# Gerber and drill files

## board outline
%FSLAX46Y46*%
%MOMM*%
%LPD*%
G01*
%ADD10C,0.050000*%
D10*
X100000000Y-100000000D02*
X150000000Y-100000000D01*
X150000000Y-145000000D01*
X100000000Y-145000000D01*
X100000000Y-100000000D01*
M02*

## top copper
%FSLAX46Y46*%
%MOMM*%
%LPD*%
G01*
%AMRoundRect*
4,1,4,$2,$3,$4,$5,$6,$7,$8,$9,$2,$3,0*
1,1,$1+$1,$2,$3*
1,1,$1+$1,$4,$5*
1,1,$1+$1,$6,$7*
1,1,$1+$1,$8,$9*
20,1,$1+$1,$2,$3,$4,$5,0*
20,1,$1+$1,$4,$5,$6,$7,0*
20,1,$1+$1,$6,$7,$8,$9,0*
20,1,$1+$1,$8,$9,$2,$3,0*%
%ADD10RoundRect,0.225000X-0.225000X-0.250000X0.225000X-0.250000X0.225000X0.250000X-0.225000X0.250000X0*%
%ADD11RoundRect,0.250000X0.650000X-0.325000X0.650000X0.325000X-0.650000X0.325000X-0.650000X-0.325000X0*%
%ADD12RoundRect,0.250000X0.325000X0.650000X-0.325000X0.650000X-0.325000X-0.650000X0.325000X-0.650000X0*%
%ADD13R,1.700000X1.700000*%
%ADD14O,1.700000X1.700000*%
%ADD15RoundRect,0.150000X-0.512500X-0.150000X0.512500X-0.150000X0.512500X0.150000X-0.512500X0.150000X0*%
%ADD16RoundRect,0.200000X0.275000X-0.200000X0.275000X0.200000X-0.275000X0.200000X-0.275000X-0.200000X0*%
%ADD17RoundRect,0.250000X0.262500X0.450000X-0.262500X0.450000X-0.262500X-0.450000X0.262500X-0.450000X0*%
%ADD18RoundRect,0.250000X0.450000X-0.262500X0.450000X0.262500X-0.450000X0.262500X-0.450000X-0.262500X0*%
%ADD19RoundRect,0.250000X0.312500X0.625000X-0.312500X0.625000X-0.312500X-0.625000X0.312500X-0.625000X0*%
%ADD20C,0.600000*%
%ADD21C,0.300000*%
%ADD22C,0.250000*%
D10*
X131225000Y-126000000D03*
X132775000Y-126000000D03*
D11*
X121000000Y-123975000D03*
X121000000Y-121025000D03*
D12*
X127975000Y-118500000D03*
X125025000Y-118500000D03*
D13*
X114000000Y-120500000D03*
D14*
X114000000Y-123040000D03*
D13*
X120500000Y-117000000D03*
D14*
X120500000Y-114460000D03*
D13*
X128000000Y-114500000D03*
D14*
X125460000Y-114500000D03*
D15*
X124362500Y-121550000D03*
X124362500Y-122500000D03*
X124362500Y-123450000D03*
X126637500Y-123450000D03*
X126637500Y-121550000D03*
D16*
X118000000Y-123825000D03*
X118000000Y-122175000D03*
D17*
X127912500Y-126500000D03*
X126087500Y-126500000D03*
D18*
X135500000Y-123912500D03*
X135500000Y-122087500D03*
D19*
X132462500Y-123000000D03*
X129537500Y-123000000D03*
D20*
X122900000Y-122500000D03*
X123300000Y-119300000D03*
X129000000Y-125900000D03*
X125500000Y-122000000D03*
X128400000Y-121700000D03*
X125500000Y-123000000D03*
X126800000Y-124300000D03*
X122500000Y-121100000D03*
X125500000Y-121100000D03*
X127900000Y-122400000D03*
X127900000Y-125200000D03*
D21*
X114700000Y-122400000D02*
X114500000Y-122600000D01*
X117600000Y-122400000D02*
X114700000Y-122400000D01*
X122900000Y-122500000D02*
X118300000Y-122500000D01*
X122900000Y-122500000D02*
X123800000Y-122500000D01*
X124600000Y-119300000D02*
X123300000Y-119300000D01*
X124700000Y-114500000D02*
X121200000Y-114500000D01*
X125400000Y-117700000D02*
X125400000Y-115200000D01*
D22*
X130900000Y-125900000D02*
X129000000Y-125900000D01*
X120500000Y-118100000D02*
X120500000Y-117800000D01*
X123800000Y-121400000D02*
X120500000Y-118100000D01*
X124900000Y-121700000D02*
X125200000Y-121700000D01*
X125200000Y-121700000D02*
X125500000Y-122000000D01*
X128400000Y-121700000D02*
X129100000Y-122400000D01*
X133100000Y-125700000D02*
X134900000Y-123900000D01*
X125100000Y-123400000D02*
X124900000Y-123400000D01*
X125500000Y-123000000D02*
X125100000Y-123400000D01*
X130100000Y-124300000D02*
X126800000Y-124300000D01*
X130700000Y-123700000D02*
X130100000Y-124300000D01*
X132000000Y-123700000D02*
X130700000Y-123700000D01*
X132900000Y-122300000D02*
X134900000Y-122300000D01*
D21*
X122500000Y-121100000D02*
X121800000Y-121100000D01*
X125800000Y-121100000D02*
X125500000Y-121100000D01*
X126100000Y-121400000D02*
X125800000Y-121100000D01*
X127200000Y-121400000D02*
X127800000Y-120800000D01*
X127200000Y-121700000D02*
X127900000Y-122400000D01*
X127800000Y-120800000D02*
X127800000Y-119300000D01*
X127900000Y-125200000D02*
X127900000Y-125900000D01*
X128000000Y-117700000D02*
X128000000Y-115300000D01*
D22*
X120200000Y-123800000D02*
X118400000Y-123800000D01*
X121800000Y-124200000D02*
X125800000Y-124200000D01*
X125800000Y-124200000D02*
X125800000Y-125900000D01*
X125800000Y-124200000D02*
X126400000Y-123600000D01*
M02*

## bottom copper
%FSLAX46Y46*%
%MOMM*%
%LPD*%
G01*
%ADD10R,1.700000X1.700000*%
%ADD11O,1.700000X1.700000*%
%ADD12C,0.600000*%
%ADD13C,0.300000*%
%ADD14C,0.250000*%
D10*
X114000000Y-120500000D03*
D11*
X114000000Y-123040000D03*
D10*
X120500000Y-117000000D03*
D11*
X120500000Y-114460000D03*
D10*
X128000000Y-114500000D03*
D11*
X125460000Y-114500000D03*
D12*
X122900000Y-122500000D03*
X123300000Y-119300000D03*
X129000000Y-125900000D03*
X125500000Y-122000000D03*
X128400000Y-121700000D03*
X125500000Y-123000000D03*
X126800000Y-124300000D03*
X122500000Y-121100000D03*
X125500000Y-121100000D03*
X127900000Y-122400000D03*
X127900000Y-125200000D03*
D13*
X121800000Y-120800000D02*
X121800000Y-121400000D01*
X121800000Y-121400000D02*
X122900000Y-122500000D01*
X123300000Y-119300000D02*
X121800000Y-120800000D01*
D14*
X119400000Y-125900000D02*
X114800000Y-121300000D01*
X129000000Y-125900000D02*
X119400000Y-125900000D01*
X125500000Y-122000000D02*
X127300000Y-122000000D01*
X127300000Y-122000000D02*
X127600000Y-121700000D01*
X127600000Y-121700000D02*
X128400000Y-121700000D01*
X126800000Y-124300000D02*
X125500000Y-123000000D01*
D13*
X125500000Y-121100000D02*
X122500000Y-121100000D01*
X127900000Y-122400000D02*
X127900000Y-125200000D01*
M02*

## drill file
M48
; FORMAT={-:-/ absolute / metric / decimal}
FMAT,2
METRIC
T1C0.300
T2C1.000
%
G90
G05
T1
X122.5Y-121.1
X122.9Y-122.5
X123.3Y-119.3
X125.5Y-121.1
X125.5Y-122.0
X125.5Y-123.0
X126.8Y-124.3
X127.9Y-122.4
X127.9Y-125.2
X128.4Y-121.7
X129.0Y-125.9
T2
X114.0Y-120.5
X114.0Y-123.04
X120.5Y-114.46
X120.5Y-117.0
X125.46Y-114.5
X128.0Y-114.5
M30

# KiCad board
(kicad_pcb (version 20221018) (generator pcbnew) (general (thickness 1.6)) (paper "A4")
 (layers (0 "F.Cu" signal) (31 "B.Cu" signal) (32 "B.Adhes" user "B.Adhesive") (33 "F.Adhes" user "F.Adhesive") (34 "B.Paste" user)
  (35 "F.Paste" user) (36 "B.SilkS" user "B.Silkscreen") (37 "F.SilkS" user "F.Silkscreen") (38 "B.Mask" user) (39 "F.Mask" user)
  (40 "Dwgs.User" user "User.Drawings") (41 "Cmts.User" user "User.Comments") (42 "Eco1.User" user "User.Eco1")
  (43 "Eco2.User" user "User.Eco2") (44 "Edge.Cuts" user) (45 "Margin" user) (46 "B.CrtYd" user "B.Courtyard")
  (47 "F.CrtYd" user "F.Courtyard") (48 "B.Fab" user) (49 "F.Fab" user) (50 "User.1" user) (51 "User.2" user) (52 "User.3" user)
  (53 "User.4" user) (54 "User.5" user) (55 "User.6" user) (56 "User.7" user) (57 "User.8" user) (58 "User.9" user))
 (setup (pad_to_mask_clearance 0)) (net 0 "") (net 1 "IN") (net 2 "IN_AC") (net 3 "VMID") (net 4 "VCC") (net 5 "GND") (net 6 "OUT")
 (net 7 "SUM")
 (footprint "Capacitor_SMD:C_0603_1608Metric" (layer "F.Cu") (at 132 126)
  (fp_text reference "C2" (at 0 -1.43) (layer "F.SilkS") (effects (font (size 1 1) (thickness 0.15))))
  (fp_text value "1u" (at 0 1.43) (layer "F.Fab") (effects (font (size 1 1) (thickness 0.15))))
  (pad "1" smd roundrect (at -0.775 0) (size 0.9 0.95) (layers "F.Cu" "F.Paste" "F.Mask") (roundrect_rratio 0.25) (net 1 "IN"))
  (pad "2" smd roundrect (at 0.775 0) (size 0.9 0.95) (layers "F.Cu" "F.Paste" "F.Mask") (roundrect_rratio 0.25) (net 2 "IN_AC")))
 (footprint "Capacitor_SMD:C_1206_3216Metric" (layer "F.Cu") (at 121 122.5 90)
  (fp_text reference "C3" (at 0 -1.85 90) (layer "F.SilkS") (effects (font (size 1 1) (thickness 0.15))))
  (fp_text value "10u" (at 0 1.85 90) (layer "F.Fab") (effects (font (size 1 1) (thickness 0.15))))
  (pad "1" smd roundrect (at -1.475 0 90) (size 1.15 1.8) (layers "F.Cu" "F.Paste" "F.Mask") (roundrect_rratio 0.217391) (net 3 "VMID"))
  (pad "2" smd roundrect (at 1.475 0 90) (size 1.15 1.8) (layers "F.Cu" "F.Paste" "F.Mask") (roundrect_rratio 0.217391) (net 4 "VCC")))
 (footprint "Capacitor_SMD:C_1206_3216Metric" (layer "F.Cu") (at 126.5 118.5 180)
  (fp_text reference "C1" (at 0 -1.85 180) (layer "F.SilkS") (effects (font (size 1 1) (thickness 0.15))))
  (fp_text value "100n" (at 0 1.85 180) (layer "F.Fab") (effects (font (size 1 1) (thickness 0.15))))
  (pad "1" smd roundrect (at -1.475 0 180) (size 1.15 1.8) (layers "F.Cu" "F.Paste" "F.Mask") (roundrect_rratio 0.217391) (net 4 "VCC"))
  (pad "2" smd roundrect (at 1.475 0 180) (size 1.15 1.8) (layers "F.Cu" "F.Paste" "F.Mask") (roundrect_rratio 0.217391) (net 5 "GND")))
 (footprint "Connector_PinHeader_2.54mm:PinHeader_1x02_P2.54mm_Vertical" (layer "F.Cu") (at 114 120.5)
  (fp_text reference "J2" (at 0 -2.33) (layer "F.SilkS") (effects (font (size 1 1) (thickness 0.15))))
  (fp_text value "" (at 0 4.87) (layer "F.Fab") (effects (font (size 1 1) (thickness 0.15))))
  (pad "1" thru_hole rect (at 0 0) (size 1.7 1.7) (drill 1) (layers "*.Cu" "*.Mask") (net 1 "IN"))
  (pad "2" thru_hole oval (at 0 2.54) (size 1.7 1.7) (drill 1) (layers "*.Cu" "*.Mask") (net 5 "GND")))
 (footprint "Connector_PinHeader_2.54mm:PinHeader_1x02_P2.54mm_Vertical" (layer "F.Cu") (at 120.5 117 180)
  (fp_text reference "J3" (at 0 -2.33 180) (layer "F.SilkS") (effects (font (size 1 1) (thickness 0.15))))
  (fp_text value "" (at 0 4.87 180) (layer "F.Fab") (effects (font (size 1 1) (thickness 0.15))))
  (pad "1" thru_hole rect (at 0 0 180) (size 1.7 1.7) (drill 1) (layers "*.Cu" "*.Mask") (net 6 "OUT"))
  (pad "2" thru_hole oval (at 0 2.54 180) (size 1.7 1.7) (drill 1) (layers "*.Cu" "*.Mask") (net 5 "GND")))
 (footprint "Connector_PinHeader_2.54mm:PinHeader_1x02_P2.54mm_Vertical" (layer "F.Cu") (at 128 114.5 -90)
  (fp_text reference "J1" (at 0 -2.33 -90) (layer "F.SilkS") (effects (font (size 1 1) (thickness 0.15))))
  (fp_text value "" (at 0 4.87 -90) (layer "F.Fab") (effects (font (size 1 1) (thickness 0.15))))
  (pad "1" thru_hole rect (at 0 0 270) (size 1.7 1.7) (drill 1) (layers "*.Cu" "*.Mask") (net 4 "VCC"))
  (pad "2" thru_hole oval (at 0 2.54 270) (size 1.7 1.7) (drill 1) (layers "*.Cu" "*.Mask") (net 5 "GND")))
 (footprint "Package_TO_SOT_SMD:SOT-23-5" (layer "F.Cu") (at 125.5 122.5)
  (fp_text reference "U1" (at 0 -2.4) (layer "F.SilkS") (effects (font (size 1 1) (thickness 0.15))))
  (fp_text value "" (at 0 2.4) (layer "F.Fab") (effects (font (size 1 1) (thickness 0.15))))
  (pad "1" smd roundrect (at -1.1375 -0.95) (size 1.325 0.6) (layers "F.Cu" "F.Paste" "F.Mask") (roundrect_rratio 0.25) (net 6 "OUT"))
  (pad "2" smd roundrect (at -1.1375 0) (size 1.325 0.6) (layers "F.Cu" "F.Paste" "F.Mask") (roundrect_rratio 0.25) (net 5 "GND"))
  (pad "3" smd roundrect (at -1.1375 0.95) (size 1.325 0.6) (layers "F.Cu" "F.Paste" "F.Mask") (roundrect_rratio 0.25) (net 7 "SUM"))
  (pad "4" smd roundrect (at 1.1375 0.95) (size 1.325 0.6) (layers "F.Cu" "F.Paste" "F.Mask") (roundrect_rratio 0.25) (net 3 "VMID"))
  (pad "5" smd roundrect (at 1.1375 -0.95) (size 1.325 0.6) (layers "F.Cu" "F.Paste" "F.Mask") (roundrect_rratio 0.25) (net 4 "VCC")))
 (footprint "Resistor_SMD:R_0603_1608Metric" (layer "F.Cu") (at 118 123 90)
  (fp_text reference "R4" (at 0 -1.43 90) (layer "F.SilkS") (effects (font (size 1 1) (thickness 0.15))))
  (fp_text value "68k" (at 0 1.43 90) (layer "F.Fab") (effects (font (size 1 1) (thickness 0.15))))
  (pad "1" smd roundrect (at -0.825 0 90) (size 0.8 0.95) (layers "F.Cu" "F.Paste" "F.Mask") (roundrect_rratio 0.25) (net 3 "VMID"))
  (pad "2" smd roundrect (at 0.825 0 90) (size 0.8 0.95) (layers "F.Cu" "F.Paste" "F.Mask") (roundrect_rratio 0.25) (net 5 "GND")))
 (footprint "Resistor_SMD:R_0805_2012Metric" (layer "F.Cu") (at 127 126.5 180)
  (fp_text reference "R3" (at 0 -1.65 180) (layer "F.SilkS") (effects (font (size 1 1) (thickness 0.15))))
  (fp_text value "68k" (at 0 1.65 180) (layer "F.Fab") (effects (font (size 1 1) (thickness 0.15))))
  (pad "1" smd roundrect (at -0.9125 0 180) (size 1.025 1.4) (layers "F.Cu" "F.Paste" "F.Mask") (roundrect_rratio 0.243902) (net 4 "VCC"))
  (pad "2" smd roundrect (at 0.9125 0 180) (size 1.025 1.4) (layers "F.Cu" "F.Paste" "F.Mask") (roundrect_rratio 0.243902) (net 3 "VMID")))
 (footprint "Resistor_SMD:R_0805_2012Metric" (layer "F.Cu") (at 135.5 123 90)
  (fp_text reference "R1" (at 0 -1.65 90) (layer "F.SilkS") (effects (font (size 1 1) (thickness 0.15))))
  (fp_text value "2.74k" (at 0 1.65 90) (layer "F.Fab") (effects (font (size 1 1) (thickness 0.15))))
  (pad "1" smd roundrect (at -0.9125 0 90) (size 1.025 1.4) (layers "F.Cu" "F.Paste" "F.Mask") (roundrect_rratio 0.243902) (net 2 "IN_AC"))
  (pad "2" smd roundrect (at 0.9125 0 90) (size 1.025 1.4) (layers "F.Cu" "F.Paste" "F.Mask") (roundrect_rratio 0.243902) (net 7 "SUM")))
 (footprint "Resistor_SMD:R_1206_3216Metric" (layer "F.Cu") (at 131 123 180)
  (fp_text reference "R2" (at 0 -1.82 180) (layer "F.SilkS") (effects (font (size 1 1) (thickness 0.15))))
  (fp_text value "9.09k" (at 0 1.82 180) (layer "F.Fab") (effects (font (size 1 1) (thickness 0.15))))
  (pad "1" smd roundrect (at -1.4625 0 180) (size 1.125 1.75) (layers "F.Cu" "F.Paste" "F.Mask") (roundrect_rratio 0.222222) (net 7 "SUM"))
  (pad "2" smd roundrect (at 1.4625 0 180) (size 1.125 1.75) (layers "F.Cu" "F.Paste" "F.Mask") (roundrect_rratio 0.222222) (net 6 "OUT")))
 (gr_rect (start 100 100) (end 150 145) (stroke (width 0.05) (type default)) (fill none) (layer "Edge.Cuts"))
 (segment (start 114.7 122.4) (end 114.5 122.6) (width 0.3) (layer "F.Cu") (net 5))
 (segment (start 117.6 122.4) (end 114.7 122.4) (width 0.3) (layer "F.Cu") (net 5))
 (segment (start 122.9 122.5) (end 118.3 122.5) (width 0.3) (layer "F.Cu") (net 5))
 (segment (start 122.9 122.5) (end 123.8 122.5) (width 0.3) (layer "F.Cu") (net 5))
 (segment (start 124.6 119.3) (end 123.3 119.3) (width 0.3) (layer "F.Cu") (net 5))
 (segment (start 124.7 114.5) (end 121.2 114.5) (width 0.3) (layer "F.Cu") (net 5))
 (segment (start 125.4 117.7) (end 125.4 115.2) (width 0.3) (layer "F.Cu") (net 5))
 (via (at 122.9 122.5) (size 0.6) (drill 0.3) (layers "F.Cu" "B.Cu") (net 5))
 (via (at 123.3 119.3) (size 0.6) (drill 0.3) (layers "F.Cu" "B.Cu") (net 5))
 (segment (start 121.8 120.8) (end 121.8 121.4) (width 0.3) (layer "B.Cu") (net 5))
 (segment (start 121.8 121.4) (end 122.9 122.5) (width 0.3) (layer "B.Cu") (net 5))
 (segment (start 123.3 119.3) (end 121.8 120.8) (width 0.3) (layer "B.Cu") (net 5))
 (segment (start 130.9 125.9) (end 129 125.9) (width 0.25) (layer "F.Cu") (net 1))
 (via (at 129 125.9) (size 0.6) (drill 0.3) (layers "F.Cu" "B.Cu") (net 1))
 (segment (start 119.4 125.9) (end 114.8 121.3) (width 0.25) (layer "B.Cu") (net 1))
 (segment (start 120.5 118.1) (end 120.5 117.8) (width 0.25) (layer "F.Cu") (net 6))
 (segment (start 123.8 121.4) (end 120.5 118.1) (width 0.25) (layer "F.Cu") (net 6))
 (segment (start 124.9 121.7) (end 125.2 121.7) (width 0.25) (layer "F.Cu") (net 6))
 (segment (start 125.2 121.7) (end 125.5 122) (width 0.25) (layer "F.Cu") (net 6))
 (segment (start 128.4 121.7) (end 129.1 122.4) (width 0.25) (layer "F.Cu") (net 6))
 (segment (start 129 125.9) (end 119.4 125.9) (width 0.25) (layer "B.Cu") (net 1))
 (segment (start 133.1 125.7) (end 134.9 123.9) (width 0.25) (layer "F.Cu") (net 2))
 (via (at 125.5 122) (size 0.6) (drill 0.3) (layers "F.Cu" "B.Cu") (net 6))
 (via (at 128.4 121.7) (size 0.6) (drill 0.3) (layers "F.Cu" "B.Cu") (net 6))
 (segment (start 125.1 123.4) (end 124.9 123.4) (width 0.25) (layer "F.Cu") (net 7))
 (segment (start 125.5 122) (end 127.3 122) (width 0.25) (layer "B.Cu") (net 6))
 (segment (start 125.5 123) (end 125.1 123.4) (width 0.25) (layer "F.Cu") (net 7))
 (segment (start 127.3 122) (end 127.6 121.7) (width 0.25) (layer "B.Cu") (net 6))
 (segment (start 127.6 121.7) (end 128.4 121.7) (width 0.25) (layer "B.Cu") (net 6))
 (segment (start 130.1 124.3) (end 126.8 124.3) (width 0.25) (layer "F.Cu") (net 7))
 (segment (start 130.7 123.7) (end 130.1 124.3) (width 0.25) (layer "F.Cu") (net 7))
 (segment (start 132 123.7) (end 130.7 123.7) (width 0.25) (layer "F.Cu") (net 7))
 (segment (start 132.9 122.3) (end 134.9 122.3) (width 0.25) (layer "F.Cu") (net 7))
 (via (at 125.5 123) (size 0.6) (drill 0.3) (layers "F.Cu" "B.Cu") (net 7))
 (via (at 126.8 124.3) (size 0.6) (drill 0.3) (layers "F.Cu" "B.Cu") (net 7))
 (segment (start 122.5 121.1) (end 121.8 121.1) (width 0.3) (layer "F.Cu") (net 4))
 (segment (start 125.8 121.1) (end 125.5 121.1) (width 0.3) (layer "F.Cu") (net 4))
 (segment (start 126.1 121.4) (end 125.8 121.1) (width 0.3) (layer "F.Cu") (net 4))
 (segment (start 126.8 124.3) (end 125.5 123) (width 0.25) (layer "B.Cu") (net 7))
 (segment (start 127.2 121.4) (end 127.8 120.8) (width 0.3) (layer "F.Cu") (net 4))
 (segment (start 127.2 121.7) (end 127.9 122.4) (width 0.3) (layer "F.Cu") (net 4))
 (segment (start 127.8 120.8) (end 127.8 119.3) (width 0.3) (layer "F.Cu") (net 4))
 (segment (start 127.9 125.2) (end 127.9 125.9) (width 0.3) (layer "F.Cu") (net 4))
 (segment (start 128 117.7) (end 128 115.3) (width 0.3) (layer "F.Cu") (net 4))
 (via (at 122.5 121.1) (size 0.6) (drill 0.3) (layers "F.Cu" "B.Cu") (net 4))
 (via (at 125.5 121.1) (size 0.6) (drill 0.3) (layers "F.Cu" "B.Cu") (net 4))
 (via (at 127.9 122.4) (size 0.6) (drill 0.3) (layers "F.Cu" "B.Cu") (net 4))
 (via (at 127.9 125.2) (size 0.6) (drill 0.3) (layers "F.Cu" "B.Cu") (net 4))
 (segment (start 120.2 123.8) (end 118.4 123.8) (width 0.25) (layer "F.Cu") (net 3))
 (segment (start 121.8 124.2) (end 125.8 124.2) (width 0.25) (layer "F.Cu") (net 3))
 (segment (start 125.5 121.1) (end 122.5 121.1) (width 0.3) (layer "B.Cu") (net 4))
 (segment (start 125.8 124.2) (end 125.8 125.9) (width 0.25) (layer "F.Cu") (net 3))
 (segment (start 125.8 124.2) (end 126.4 123.6) (width 0.25) (layer "F.Cu") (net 3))
 (segment (start 127.9 122.4) (end 127.9 125.2) (width 0.3) (layer "B.Cu") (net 4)))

